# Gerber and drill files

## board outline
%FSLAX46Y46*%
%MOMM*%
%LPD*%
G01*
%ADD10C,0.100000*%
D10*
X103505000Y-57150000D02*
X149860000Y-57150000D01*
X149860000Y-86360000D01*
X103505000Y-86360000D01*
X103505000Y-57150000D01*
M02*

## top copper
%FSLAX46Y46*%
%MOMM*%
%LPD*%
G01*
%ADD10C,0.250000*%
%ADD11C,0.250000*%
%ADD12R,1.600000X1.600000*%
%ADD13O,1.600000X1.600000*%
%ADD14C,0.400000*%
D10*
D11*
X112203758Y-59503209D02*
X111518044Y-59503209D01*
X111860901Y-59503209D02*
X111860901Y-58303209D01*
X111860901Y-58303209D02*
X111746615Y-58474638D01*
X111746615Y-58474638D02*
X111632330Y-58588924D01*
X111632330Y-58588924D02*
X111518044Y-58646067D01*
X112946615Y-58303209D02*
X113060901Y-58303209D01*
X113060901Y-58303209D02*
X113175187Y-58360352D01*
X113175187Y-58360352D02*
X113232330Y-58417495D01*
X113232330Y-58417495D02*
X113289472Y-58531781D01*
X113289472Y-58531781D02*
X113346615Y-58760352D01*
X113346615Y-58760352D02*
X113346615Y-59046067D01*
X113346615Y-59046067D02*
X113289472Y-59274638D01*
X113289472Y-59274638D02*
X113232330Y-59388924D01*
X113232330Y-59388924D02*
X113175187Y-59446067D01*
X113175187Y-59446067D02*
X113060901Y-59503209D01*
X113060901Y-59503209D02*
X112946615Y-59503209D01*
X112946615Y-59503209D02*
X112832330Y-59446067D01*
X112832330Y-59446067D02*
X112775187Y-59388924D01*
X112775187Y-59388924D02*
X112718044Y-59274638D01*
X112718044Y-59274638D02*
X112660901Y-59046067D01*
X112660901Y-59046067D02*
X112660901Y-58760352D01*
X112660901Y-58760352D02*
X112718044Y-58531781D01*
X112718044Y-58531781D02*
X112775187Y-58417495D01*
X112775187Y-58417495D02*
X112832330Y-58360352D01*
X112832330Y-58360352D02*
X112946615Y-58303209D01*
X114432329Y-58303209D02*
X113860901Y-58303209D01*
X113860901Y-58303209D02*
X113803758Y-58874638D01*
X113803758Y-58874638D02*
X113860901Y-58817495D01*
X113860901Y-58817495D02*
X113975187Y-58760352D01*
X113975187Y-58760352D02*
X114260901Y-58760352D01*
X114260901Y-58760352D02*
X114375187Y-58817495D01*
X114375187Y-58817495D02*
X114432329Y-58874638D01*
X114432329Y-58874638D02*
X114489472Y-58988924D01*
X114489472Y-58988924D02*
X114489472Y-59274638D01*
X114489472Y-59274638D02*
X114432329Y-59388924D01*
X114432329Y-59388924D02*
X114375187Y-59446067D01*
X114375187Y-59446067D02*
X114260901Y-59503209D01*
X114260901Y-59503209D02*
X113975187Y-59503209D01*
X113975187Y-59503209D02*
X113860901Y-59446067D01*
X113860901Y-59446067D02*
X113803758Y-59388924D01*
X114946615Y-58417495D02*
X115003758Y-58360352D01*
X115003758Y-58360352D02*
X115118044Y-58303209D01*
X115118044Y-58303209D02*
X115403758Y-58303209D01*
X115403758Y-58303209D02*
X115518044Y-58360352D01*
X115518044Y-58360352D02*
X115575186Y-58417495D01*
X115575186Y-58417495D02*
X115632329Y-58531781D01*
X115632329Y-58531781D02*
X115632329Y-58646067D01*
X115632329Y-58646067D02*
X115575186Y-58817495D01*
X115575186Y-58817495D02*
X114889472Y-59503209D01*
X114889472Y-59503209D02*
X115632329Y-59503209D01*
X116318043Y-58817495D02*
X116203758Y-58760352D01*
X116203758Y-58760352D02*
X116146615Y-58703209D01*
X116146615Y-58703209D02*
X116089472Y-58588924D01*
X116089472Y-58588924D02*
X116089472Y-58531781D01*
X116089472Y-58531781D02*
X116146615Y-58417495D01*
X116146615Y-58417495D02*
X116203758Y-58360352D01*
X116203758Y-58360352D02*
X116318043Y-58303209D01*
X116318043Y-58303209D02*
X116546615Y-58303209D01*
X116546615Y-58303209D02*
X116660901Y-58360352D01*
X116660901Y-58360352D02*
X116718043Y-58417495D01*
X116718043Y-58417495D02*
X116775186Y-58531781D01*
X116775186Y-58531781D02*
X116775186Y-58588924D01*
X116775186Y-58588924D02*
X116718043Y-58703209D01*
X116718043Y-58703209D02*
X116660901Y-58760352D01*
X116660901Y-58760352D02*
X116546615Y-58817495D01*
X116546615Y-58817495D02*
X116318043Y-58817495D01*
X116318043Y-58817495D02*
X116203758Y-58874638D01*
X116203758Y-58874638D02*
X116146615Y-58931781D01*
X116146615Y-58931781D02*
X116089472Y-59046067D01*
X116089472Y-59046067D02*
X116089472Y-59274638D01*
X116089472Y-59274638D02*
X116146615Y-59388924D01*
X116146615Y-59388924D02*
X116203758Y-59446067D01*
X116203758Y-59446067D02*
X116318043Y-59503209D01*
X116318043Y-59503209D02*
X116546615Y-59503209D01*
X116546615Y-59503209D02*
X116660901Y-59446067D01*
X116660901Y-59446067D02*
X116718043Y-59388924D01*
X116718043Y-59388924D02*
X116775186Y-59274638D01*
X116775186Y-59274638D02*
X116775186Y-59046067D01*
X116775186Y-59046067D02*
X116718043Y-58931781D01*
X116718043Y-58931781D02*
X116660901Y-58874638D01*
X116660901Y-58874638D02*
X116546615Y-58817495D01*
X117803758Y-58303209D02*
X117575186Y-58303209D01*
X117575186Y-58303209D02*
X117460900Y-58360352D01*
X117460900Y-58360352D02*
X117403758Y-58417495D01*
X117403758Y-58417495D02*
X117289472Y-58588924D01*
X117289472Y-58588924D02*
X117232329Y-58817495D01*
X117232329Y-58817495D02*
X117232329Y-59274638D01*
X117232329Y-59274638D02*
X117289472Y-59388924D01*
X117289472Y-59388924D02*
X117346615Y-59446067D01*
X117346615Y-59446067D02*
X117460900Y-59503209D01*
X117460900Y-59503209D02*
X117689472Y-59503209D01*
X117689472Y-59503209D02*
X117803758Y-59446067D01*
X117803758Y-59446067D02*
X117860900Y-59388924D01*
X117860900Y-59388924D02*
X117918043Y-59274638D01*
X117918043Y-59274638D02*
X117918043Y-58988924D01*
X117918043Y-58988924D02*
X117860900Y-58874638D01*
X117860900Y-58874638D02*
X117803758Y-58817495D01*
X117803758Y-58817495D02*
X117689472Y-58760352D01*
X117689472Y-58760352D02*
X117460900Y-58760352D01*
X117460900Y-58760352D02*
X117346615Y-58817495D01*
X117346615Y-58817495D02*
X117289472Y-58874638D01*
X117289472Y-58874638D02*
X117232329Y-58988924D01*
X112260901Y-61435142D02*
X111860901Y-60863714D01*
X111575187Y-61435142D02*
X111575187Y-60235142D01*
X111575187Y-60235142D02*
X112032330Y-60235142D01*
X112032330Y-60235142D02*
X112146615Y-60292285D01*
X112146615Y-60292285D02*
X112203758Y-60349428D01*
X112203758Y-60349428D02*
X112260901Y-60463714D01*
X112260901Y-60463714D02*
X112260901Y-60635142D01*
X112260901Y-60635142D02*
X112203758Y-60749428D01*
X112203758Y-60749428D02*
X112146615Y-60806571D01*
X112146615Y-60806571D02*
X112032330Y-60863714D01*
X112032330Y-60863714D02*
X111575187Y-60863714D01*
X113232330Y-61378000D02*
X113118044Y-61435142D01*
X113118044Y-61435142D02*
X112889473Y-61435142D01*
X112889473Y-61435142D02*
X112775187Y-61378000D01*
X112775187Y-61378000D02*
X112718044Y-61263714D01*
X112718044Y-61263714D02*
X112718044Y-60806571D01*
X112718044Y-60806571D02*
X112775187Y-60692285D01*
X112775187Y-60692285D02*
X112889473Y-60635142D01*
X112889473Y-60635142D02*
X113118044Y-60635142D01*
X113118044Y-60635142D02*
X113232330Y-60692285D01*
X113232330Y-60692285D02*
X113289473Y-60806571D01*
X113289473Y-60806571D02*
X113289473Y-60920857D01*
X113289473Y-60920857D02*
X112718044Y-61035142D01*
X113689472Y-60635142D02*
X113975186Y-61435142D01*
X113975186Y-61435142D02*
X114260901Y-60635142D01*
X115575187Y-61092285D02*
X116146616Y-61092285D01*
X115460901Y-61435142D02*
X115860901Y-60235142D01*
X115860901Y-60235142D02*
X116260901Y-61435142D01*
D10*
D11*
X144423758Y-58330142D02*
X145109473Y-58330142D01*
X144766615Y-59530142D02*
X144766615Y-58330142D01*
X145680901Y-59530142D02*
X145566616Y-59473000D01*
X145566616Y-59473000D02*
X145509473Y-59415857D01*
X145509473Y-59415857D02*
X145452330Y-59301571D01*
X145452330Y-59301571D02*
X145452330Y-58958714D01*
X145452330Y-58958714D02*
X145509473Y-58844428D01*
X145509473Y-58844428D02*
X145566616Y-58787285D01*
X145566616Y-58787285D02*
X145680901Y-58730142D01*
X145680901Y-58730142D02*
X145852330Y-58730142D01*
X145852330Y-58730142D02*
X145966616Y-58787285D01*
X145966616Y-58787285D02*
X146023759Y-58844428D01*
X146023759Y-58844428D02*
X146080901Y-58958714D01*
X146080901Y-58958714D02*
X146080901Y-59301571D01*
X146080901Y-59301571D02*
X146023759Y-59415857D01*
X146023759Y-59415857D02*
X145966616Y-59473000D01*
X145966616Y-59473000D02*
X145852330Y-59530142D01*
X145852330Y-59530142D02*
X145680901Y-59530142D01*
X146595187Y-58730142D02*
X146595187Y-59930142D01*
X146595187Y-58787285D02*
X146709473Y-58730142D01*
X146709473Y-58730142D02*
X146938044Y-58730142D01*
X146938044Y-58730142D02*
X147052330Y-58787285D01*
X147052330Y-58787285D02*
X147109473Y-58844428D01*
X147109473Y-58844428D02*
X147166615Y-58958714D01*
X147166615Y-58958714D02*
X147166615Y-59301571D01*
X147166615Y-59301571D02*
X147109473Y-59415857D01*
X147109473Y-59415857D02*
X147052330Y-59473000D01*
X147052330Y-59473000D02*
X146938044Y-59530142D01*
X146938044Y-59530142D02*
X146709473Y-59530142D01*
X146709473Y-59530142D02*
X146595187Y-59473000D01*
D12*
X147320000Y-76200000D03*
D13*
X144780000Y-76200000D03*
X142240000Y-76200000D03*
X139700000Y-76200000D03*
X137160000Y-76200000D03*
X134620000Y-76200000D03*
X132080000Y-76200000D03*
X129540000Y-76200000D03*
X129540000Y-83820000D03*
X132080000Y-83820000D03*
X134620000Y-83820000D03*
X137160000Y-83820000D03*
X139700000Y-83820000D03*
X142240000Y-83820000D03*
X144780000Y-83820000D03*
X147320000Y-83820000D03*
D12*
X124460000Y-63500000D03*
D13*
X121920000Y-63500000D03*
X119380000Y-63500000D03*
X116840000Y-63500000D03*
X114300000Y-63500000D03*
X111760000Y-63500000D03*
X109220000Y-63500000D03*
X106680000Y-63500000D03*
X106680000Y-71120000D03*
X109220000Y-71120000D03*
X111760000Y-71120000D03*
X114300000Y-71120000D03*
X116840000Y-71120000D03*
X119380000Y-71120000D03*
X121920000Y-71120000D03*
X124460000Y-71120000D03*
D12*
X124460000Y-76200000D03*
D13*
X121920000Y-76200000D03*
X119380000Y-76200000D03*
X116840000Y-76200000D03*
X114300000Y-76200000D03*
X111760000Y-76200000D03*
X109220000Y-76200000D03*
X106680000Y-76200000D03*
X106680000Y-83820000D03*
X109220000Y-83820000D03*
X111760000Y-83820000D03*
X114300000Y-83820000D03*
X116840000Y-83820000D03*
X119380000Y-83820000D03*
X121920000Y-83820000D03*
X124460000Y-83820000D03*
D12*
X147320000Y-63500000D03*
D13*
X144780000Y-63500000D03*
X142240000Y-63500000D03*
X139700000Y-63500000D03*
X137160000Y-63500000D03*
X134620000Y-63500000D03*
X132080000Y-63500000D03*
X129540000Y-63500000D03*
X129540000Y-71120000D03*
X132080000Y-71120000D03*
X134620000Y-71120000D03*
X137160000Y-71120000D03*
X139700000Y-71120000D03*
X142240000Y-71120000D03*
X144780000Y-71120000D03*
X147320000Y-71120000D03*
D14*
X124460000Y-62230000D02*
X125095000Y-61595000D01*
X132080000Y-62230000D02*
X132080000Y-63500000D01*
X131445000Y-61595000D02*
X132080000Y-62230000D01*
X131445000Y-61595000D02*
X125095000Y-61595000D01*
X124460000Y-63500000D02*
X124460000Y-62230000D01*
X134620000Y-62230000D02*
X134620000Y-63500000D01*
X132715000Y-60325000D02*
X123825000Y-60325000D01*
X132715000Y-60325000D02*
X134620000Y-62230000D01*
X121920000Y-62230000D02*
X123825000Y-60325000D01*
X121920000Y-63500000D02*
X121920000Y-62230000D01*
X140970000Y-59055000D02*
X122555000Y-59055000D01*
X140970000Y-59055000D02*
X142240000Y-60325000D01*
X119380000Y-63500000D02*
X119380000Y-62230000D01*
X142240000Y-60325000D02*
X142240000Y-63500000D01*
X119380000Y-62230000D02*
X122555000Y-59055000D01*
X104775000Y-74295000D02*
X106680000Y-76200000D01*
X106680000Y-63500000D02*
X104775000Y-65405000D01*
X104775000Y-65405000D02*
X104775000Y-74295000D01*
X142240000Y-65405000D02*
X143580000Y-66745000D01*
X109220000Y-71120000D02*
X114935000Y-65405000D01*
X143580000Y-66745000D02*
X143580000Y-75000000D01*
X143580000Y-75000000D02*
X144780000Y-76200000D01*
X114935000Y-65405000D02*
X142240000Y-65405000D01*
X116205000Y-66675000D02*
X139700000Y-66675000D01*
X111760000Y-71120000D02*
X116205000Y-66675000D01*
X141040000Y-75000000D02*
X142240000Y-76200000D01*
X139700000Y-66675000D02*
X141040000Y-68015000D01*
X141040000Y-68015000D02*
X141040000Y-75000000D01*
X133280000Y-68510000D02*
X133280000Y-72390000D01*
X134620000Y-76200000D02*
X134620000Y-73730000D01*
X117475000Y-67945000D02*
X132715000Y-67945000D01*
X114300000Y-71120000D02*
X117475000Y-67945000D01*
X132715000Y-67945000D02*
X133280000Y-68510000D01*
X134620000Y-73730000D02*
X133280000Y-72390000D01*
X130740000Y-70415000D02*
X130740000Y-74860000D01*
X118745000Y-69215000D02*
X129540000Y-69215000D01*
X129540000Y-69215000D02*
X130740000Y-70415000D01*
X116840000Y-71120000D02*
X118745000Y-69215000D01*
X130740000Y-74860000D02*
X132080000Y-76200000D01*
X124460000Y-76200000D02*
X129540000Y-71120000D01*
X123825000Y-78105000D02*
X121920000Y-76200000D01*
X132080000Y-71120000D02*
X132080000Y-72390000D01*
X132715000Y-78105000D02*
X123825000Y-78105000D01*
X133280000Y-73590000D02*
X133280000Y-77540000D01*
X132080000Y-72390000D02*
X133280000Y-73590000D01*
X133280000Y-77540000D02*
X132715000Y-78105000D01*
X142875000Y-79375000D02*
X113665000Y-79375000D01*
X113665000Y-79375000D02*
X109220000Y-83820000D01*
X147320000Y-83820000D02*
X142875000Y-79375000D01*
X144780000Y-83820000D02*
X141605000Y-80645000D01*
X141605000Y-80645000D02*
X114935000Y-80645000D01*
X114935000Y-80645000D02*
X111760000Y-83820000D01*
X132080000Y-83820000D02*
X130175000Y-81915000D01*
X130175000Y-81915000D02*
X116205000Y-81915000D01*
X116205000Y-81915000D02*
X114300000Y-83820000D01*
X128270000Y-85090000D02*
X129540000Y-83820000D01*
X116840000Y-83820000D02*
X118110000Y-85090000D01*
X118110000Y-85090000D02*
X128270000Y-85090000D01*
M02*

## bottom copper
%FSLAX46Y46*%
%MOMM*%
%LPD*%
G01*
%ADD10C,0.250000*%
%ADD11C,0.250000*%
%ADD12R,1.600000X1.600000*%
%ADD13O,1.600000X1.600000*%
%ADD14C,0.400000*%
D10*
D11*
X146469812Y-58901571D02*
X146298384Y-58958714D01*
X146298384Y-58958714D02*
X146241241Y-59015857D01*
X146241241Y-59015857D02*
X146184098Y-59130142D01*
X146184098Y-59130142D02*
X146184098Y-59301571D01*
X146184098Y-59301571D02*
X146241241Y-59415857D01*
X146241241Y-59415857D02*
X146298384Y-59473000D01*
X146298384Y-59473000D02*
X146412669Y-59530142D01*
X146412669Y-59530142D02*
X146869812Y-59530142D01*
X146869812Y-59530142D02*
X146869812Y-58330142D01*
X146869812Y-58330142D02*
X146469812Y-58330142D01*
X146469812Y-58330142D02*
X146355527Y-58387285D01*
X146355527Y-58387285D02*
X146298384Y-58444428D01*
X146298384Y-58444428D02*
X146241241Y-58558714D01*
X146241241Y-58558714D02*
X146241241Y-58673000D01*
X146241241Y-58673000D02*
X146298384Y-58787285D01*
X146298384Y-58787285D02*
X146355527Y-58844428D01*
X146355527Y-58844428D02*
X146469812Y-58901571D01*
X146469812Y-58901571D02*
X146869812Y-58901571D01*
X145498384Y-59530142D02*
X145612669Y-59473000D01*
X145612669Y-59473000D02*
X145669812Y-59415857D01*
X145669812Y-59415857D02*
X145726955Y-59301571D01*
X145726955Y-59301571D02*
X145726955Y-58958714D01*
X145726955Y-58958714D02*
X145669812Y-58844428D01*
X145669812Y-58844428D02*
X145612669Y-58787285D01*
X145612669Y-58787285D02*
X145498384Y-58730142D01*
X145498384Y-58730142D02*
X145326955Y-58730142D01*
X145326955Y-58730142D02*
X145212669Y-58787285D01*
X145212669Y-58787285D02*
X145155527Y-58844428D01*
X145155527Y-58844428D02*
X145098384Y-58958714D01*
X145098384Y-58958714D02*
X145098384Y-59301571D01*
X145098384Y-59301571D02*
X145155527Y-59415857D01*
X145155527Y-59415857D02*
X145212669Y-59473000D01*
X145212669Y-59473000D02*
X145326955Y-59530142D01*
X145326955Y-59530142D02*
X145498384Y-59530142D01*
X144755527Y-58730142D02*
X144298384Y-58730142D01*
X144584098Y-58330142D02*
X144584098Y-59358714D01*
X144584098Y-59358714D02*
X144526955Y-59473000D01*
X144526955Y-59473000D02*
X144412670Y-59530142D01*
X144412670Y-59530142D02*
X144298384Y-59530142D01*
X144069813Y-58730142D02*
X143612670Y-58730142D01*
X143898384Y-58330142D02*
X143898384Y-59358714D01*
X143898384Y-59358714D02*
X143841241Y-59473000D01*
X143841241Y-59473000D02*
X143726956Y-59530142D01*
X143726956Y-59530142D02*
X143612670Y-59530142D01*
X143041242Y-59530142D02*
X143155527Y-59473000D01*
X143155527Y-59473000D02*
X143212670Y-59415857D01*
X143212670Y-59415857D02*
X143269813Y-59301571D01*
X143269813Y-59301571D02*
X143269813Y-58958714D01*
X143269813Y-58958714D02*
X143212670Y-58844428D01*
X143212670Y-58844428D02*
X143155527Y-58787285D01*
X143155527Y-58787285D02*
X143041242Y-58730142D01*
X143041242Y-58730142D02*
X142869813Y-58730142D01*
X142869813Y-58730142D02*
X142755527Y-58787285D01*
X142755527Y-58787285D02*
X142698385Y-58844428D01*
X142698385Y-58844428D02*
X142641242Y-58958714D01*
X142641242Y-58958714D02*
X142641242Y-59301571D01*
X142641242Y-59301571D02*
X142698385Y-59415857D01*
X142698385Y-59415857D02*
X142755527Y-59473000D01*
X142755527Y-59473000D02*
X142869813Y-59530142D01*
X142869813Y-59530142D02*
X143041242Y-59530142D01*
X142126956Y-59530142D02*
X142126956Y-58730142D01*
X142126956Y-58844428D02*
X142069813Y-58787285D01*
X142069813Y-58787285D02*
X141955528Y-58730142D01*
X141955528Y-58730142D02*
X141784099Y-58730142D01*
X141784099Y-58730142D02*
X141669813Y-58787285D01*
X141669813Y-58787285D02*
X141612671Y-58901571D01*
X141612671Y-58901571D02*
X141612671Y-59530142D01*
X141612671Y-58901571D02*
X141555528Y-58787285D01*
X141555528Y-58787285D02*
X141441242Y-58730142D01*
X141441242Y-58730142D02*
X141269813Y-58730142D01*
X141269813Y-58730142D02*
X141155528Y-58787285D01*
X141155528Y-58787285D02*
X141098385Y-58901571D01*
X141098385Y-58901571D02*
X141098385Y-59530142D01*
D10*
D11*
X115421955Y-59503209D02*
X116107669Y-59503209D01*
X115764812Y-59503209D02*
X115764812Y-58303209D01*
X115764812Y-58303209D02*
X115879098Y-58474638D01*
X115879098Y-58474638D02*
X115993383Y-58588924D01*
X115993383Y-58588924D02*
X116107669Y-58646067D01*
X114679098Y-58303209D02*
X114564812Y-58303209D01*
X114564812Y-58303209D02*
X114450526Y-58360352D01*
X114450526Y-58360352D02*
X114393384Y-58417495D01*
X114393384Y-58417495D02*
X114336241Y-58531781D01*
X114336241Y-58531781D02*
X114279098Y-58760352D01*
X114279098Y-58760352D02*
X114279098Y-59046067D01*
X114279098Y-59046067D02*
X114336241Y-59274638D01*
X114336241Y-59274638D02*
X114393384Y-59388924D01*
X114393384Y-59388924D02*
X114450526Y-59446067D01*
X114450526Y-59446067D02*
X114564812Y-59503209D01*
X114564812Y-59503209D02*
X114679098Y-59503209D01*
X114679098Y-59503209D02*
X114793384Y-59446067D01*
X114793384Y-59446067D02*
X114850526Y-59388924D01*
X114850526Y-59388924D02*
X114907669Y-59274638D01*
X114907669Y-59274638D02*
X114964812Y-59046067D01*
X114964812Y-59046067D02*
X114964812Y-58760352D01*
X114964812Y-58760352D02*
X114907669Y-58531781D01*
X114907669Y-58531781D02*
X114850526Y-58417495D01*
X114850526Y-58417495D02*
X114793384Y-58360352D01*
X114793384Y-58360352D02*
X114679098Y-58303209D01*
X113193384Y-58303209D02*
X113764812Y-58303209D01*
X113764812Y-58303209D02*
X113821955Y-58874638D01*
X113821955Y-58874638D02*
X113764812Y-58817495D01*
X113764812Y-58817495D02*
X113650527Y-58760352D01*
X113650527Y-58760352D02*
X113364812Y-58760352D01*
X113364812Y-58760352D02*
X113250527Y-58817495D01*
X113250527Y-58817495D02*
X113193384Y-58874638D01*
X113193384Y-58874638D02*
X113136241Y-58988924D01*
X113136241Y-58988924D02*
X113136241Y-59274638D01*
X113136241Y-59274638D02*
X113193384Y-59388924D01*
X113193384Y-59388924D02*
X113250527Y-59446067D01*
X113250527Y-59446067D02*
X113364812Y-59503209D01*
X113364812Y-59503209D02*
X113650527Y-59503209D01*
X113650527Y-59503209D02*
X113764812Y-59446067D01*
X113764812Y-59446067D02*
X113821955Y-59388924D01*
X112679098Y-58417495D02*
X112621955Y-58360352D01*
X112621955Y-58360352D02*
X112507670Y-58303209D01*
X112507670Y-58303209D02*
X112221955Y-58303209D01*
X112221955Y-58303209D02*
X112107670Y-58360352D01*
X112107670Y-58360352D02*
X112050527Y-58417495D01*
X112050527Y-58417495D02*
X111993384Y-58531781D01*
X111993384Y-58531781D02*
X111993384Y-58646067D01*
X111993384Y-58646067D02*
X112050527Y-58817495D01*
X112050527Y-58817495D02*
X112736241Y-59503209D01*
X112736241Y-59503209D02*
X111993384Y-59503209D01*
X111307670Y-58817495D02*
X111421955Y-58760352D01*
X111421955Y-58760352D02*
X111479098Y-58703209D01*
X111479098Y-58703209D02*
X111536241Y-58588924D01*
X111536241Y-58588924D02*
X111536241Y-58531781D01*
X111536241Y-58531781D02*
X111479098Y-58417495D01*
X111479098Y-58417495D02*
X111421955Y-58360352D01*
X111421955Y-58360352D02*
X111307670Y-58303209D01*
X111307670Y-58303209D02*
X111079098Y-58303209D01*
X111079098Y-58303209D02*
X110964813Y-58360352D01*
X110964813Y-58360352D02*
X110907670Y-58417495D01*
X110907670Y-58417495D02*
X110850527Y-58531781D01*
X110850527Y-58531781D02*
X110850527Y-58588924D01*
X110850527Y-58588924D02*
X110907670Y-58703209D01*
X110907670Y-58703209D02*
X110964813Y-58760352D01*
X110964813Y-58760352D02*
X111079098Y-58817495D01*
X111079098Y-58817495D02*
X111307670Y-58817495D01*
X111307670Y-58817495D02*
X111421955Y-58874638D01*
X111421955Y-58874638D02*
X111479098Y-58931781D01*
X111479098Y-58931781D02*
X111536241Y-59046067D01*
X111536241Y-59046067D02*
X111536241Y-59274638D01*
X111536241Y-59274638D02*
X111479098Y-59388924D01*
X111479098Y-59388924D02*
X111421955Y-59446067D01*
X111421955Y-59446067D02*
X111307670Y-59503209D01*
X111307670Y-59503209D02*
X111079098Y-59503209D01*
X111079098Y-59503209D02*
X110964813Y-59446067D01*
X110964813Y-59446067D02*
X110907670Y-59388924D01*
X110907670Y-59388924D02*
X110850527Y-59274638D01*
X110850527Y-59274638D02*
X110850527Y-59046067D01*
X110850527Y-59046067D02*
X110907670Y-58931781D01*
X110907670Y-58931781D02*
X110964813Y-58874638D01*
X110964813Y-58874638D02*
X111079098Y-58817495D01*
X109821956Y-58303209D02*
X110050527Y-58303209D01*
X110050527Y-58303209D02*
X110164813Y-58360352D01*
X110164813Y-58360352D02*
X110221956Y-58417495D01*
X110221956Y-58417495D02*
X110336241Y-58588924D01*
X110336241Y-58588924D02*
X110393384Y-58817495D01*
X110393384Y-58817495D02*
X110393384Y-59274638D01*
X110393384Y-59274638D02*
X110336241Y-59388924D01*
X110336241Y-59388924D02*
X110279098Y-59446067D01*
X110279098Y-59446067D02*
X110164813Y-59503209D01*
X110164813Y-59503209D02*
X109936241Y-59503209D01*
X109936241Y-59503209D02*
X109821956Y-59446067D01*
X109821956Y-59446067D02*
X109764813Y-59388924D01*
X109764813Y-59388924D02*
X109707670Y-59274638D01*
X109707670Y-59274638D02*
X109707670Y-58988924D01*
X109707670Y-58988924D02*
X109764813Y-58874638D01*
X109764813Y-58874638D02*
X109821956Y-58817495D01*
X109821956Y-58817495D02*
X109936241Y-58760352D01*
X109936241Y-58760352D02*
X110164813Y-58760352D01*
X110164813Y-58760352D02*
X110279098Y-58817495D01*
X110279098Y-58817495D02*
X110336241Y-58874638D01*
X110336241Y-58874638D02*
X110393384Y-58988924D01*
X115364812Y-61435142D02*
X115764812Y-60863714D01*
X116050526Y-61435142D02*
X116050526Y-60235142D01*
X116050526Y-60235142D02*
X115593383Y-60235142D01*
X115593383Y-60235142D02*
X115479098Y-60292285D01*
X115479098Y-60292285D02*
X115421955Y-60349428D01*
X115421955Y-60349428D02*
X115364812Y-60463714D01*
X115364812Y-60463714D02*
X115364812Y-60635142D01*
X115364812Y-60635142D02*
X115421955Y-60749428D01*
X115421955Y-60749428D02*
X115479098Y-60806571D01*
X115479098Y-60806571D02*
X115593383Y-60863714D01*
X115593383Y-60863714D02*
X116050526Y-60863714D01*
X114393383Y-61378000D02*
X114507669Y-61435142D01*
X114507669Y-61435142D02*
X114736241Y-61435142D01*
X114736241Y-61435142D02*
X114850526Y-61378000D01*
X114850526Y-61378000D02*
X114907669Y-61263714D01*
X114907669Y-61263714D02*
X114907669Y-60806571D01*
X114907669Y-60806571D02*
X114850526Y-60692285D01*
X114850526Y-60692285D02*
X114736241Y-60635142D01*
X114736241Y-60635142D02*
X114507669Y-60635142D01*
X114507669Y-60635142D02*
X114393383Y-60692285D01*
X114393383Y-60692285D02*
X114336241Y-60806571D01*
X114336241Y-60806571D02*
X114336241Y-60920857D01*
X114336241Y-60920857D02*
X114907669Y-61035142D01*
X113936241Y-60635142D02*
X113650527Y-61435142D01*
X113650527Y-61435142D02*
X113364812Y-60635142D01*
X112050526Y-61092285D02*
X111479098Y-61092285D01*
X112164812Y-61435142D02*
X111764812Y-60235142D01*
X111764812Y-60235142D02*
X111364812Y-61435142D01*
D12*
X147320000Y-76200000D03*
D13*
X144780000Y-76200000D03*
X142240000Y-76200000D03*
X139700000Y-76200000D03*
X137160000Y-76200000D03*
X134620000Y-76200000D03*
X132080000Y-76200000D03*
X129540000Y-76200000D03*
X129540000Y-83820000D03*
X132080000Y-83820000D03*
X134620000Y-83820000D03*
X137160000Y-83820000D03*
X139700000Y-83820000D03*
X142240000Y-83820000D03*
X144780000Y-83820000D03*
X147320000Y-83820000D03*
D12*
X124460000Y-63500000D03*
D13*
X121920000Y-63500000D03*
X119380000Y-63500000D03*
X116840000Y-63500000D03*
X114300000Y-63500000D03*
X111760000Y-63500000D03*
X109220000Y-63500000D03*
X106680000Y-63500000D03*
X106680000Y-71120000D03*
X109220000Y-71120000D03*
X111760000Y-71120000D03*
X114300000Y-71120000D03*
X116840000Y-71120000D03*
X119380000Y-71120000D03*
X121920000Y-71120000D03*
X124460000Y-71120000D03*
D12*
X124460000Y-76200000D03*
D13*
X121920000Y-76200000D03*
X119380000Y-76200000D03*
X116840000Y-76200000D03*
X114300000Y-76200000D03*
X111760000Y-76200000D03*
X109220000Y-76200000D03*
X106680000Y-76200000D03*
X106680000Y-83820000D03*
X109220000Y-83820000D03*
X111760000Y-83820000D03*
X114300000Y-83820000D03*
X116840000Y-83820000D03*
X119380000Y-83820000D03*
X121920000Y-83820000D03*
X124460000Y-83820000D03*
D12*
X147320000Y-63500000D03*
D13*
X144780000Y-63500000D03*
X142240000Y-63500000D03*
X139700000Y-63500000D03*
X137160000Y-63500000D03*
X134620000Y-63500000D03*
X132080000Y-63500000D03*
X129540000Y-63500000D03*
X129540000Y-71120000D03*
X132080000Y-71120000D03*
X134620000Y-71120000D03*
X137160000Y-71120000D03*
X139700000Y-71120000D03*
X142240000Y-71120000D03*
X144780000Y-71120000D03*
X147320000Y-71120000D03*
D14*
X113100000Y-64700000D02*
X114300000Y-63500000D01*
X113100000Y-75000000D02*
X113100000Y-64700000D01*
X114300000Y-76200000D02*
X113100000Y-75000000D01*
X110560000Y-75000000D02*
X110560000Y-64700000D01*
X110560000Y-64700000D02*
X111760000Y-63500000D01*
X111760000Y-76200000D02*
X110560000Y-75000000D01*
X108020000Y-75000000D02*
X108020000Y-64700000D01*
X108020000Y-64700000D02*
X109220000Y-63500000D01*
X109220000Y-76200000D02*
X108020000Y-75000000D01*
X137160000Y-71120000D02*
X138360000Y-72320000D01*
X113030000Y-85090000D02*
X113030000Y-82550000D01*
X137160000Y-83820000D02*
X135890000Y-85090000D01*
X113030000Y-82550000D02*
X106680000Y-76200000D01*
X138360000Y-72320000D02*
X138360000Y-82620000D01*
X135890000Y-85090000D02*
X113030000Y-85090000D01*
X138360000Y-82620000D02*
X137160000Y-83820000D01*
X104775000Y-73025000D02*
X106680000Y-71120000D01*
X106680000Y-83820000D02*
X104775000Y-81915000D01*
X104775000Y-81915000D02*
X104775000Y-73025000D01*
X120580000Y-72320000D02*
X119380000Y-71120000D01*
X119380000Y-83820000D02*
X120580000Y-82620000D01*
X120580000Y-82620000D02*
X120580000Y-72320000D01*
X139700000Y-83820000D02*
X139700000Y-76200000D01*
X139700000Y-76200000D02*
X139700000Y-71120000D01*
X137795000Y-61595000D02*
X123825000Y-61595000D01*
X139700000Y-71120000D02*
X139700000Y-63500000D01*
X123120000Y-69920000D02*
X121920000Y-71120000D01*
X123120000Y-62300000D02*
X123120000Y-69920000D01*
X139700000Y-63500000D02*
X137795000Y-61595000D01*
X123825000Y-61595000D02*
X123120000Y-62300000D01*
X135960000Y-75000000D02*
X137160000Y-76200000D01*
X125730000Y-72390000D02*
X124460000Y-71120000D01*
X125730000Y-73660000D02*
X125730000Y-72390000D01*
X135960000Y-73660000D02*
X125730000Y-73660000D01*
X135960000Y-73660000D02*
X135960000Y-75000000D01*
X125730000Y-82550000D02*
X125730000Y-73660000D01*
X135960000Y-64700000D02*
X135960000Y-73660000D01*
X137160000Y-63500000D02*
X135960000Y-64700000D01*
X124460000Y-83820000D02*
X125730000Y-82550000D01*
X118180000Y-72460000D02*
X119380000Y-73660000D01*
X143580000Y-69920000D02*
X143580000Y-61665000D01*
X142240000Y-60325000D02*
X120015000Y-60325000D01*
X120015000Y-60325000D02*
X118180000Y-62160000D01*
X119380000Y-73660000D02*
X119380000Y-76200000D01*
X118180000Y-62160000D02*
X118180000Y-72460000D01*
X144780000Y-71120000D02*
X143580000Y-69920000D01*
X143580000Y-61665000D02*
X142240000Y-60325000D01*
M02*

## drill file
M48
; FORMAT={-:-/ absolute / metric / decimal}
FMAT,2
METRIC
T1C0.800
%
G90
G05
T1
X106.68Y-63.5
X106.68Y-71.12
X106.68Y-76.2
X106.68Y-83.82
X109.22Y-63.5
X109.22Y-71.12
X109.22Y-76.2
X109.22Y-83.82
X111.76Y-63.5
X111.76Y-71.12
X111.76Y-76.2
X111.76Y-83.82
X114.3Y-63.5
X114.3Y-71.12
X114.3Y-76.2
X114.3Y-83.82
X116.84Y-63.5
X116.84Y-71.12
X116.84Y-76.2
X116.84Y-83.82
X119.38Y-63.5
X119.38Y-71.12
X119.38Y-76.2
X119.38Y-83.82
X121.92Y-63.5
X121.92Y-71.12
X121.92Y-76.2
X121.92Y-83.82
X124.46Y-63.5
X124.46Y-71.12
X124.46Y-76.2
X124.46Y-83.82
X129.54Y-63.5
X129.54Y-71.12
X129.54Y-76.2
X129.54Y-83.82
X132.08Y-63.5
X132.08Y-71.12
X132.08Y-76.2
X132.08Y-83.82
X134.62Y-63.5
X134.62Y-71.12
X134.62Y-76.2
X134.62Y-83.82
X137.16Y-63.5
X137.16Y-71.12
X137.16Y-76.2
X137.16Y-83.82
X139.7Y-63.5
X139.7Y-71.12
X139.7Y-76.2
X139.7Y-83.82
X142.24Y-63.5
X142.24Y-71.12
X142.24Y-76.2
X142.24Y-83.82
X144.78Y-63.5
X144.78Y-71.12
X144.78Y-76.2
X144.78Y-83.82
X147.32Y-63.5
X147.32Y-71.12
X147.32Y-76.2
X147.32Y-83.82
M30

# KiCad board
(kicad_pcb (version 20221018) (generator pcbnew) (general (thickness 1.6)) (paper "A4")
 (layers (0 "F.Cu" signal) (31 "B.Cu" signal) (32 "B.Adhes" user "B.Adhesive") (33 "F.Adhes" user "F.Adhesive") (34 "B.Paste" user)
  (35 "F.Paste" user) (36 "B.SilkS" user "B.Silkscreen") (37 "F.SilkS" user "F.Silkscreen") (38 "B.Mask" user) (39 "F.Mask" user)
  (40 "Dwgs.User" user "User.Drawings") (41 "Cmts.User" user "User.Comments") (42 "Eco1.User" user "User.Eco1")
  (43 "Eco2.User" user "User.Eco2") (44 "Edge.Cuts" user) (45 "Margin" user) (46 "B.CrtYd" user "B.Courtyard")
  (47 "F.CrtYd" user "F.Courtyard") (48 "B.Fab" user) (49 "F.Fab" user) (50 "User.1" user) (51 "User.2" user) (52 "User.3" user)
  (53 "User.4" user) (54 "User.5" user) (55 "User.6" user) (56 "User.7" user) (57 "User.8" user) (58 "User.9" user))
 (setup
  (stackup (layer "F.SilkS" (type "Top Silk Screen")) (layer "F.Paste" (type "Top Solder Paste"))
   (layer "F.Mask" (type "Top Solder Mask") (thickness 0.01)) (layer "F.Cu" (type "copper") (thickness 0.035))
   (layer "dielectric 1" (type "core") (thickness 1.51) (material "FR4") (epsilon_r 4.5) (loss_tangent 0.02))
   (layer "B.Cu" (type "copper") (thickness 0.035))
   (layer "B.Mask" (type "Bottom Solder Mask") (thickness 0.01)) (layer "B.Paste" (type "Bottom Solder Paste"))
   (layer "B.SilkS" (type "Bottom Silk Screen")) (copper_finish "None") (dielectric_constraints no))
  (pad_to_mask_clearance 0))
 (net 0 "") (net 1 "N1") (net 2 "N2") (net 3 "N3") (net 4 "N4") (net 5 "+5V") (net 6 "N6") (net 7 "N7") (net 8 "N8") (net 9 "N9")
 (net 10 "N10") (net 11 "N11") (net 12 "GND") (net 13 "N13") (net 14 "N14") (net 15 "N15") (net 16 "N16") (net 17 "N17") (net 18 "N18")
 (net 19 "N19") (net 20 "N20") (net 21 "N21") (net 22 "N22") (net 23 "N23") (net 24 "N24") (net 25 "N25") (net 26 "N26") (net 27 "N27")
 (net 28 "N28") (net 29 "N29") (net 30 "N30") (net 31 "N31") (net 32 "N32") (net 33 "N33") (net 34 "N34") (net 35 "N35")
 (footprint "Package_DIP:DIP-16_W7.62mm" (layer "F.Cu") (at 147.32 76.2 -90)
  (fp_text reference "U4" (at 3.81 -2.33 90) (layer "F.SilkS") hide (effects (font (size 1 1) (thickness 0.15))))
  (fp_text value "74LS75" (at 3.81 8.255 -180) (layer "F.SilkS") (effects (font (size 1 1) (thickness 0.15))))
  (pad "1" thru_hole rect (at 0 0 270) (size 1.6 1.6) (drill 0.8) (layers "*.Cu" "*.Mask") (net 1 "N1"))
  (pad "2" thru_hole oval (at 0 2.54 270) (size 1.6 1.6) (drill 0.8) (layers "*.Cu" "*.Mask") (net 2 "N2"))
  (pad "3" thru_hole oval (at 0 5.08 270) (size 1.6 1.6) (drill 0.8) (layers "*.Cu" "*.Mask") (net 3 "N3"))
  (pad "4" thru_hole oval (at 0 7.62 270) (size 1.6 1.6) (drill 0.8) (layers "*.Cu" "*.Mask") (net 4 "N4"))
  (pad "5" thru_hole oval (at 0 10.16 270) (size 1.6 1.6) (drill 0.8) (layers "*.Cu" "*.Mask") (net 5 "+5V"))
  (pad "6" thru_hole oval (at 0 12.7 270) (size 1.6 1.6) (drill 0.8) (layers "*.Cu" "*.Mask") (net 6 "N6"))
  (pad "7" thru_hole oval (at 0 15.24 270) (size 1.6 1.6) (drill 0.8) (layers "*.Cu" "*.Mask") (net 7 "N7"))
  (pad "8" thru_hole oval (at 0 17.78 270) (size 1.6 1.6) (drill 0.8) (layers "*.Cu" "*.Mask") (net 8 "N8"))
  (pad "9" thru_hole oval (at 7.62 17.78 270) (size 1.6 1.6) (drill 0.8) (layers "*.Cu" "*.Mask") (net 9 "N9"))
  (pad "10" thru_hole oval (at 7.62 15.24 270) (size 1.6 1.6) (drill 0.8) (layers "*.Cu" "*.Mask") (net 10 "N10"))
  (pad "11" thru_hole oval (at 7.62 12.7 270) (size 1.6 1.6) (drill 0.8) (layers "*.Cu" "*.Mask") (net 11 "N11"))
  (pad "12" thru_hole oval (at 7.62 10.16 270) (size 1.6 1.6) (drill 0.8) (layers "*.Cu" "*.Mask") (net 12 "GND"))
  (pad "13" thru_hole oval (at 7.62 7.62 270) (size 1.6 1.6) (drill 0.8) (layers "*.Cu" "*.Mask") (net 4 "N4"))
  (pad "14" thru_hole oval (at 7.62 5.08 270) (size 1.6 1.6) (drill 0.8) (layers "*.Cu" "*.Mask") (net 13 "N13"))
  (pad "15" thru_hole oval (at 7.62 2.54 270) (size 1.6 1.6) (drill 0.8) (layers "*.Cu" "*.Mask") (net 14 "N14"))
  (pad "16" thru_hole oval (at 7.62 0 270) (size 1.6 1.6) (drill 0.8) (layers "*.Cu" "*.Mask") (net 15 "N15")))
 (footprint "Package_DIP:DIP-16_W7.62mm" (layer "F.Cu") (at 124.46 63.5 -90)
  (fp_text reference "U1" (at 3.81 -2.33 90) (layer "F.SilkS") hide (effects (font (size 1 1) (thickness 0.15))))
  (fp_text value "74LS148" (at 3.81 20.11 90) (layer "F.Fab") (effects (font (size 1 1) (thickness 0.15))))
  (pad "1" thru_hole rect (at 0 0 270) (size 1.6 1.6) (drill 0.8) (layers "*.Cu" "*.Mask") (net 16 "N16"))
  (pad "2" thru_hole oval (at 0 2.54 270) (size 1.6 1.6) (drill 0.8) (layers "*.Cu" "*.Mask") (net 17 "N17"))
  (pad "3" thru_hole oval (at 0 5.08 270) (size 1.6 1.6) (drill 0.8) (layers "*.Cu" "*.Mask") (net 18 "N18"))
  (pad "4" thru_hole oval (at 0 7.62 270) (size 1.6 1.6) (drill 0.8) (layers "*.Cu" "*.Mask") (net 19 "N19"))
  (pad "5" thru_hole oval (at 0 10.16 270) (size 1.6 1.6) (drill 0.8) (layers "*.Cu" "*.Mask") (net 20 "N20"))
  (pad "6" thru_hole oval (at 0 12.7 270) (size 1.6 1.6) (drill 0.8) (layers "*.Cu" "*.Mask") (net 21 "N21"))
  (pad "7" thru_hole oval (at 0 15.24 270) (size 1.6 1.6) (drill 0.8) (layers "*.Cu" "*.Mask") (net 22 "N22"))
  (pad "8" thru_hole oval (at 0 17.78 270) (size 1.6 1.6) (drill 0.8) (layers "*.Cu" "*.Mask") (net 12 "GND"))
  (pad "9" thru_hole oval (at 7.62 17.78 270) (size 1.6 1.6) (drill 0.8) (layers "*.Cu" "*.Mask") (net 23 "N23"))
  (pad "10" thru_hole oval (at 7.62 15.24 270) (size 1.6 1.6) (drill 0.8) (layers "*.Cu" "*.Mask") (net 2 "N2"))
  (pad "11" thru_hole oval (at 7.62 12.7 270) (size 1.6 1.6) (drill 0.8) (layers "*.Cu" "*.Mask") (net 3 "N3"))
  (pad "12" thru_hole oval (at 7.62 10.16 270) (size 1.6 1.6) (drill 0.8) (layers "*.Cu" "*.Mask") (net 6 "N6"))
  (pad "13" thru_hole oval (at 7.62 7.62 270) (size 1.6 1.6) (drill 0.8) (layers "*.Cu" "*.Mask") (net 7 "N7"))
  (pad "14" thru_hole oval (at 7.62 5.08 270) (size 1.6 1.6) (drill 0.8) (layers "*.Cu" "*.Mask") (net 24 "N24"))
  (pad "15" thru_hole oval (at 7.62 2.54 270) (size 1.6 1.6) (drill 0.8) (layers "*.Cu" "*.Mask") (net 4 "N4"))
  (pad "16" thru_hole oval (at 7.62 0 270) (size 1.6 1.6) (drill 0.8) (layers "*.Cu" "*.Mask") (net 5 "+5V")))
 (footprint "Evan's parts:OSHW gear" (layer "F.Cu") (at 108.585 80.01)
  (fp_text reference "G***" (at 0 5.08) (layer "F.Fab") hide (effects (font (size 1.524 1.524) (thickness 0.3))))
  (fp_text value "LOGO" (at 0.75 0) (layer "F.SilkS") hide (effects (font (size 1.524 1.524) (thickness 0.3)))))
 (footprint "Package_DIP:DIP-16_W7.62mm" (layer "F.Cu") (at 124.46 76.2 -90)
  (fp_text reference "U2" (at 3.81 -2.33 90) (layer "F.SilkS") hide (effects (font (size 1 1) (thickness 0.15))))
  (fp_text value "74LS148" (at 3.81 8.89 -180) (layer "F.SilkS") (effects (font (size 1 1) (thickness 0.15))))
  (pad "1" thru_hole rect (at 0 0 270) (size 1.6 1.6) (drill 0.8) (layers "*.Cu" "*.Mask") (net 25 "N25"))
  (pad "2" thru_hole oval (at 0 2.54 270) (size 1.6 1.6) (drill 0.8) (layers "*.Cu" "*.Mask") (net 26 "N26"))
  (pad "3" thru_hole oval (at 0 5.08 270) (size 1.6 1.6) (drill 0.8) (layers "*.Cu" "*.Mask") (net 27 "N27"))
  (pad "4" thru_hole oval (at 0 7.62 270) (size 1.6 1.6) (drill 0.8) (layers "*.Cu" "*.Mask") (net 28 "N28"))
  (pad "5" thru_hole oval (at 0 10.16 270) (size 1.6 1.6) (drill 0.8) (layers "*.Cu" "*.Mask") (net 20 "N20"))
  (pad "6" thru_hole oval (at 0 12.7 270) (size 1.6 1.6) (drill 0.8) (layers "*.Cu" "*.Mask") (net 21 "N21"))
  (pad "7" thru_hole oval (at 0 15.24 270) (size 1.6 1.6) (drill 0.8) (layers "*.Cu" "*.Mask") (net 22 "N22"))
  (pad "8" thru_hole oval (at 0 17.78 270) (size 1.6 1.6) (drill 0.8) (layers "*.Cu" "*.Mask") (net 12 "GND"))
  (pad "9" thru_hole oval (at 7.62 17.78 270) (size 1.6 1.6) (drill 0.8) (layers "*.Cu" "*.Mask") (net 23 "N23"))
  (pad "10" thru_hole oval (at 7.62 15.24 270) (size 1.6 1.6) (drill 0.8) (layers "*.Cu" "*.Mask") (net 15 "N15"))
  (pad "11" thru_hole oval (at 7.62 12.7 270) (size 1.6 1.6) (drill 0.8) (layers "*.Cu" "*.Mask") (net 14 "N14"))
  (pad "12" thru_hole oval (at 7.62 10.16 270) (size 1.6 1.6) (drill 0.8) (layers "*.Cu" "*.Mask") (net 10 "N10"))
  (pad "13" thru_hole oval (at 7.62 7.62 270) (size 1.6 1.6) (drill 0.8) (layers "*.Cu" "*.Mask") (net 9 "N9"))
  (pad "14" thru_hole oval (at 7.62 5.08 270) (size 1.6 1.6) (drill 0.8) (layers "*.Cu" "*.Mask") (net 24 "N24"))
  (pad "15" thru_hole oval (at 7.62 2.54 270) (size 1.6 1.6) (drill 0.8) (layers "*.Cu" "*.Mask") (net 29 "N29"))
  (pad "16" thru_hole oval (at 7.62 0 270) (size 1.6 1.6) (drill 0.8) (layers "*.Cu" "*.Mask") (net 5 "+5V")))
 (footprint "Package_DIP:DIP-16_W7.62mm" (layer "F.Cu") (at 147.32 63.5 -90)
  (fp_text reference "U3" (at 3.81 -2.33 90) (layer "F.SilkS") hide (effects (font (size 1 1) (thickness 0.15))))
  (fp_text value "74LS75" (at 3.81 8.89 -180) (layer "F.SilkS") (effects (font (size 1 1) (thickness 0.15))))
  (pad "1" thru_hole rect (at 0 0 270) (size 1.6 1.6) (drill 0.8) (layers "*.Cu" "*.Mask") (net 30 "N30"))
  (pad "2" thru_hole oval (at 0 2.54 270) (size 1.6 1.6) (drill 0.8) (layers "*.Cu" "*.Mask") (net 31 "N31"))
  (pad "3" thru_hole oval (at 0 5.08 270) (size 1.6 1.6) (drill 0.8) (layers "*.Cu" "*.Mask") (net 18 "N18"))
  (pad "4" thru_hole oval (at 0 7.62 270) (size 1.6 1.6) (drill 0.8) (layers "*.Cu" "*.Mask") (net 4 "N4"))
  (pad "5" thru_hole oval (at 0 10.16 270) (size 1.6 1.6) (drill 0.8) (layers "*.Cu" "*.Mask") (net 5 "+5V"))
  (pad "6" thru_hole oval (at 0 12.7 270) (size 1.6 1.6) (drill 0.8) (layers "*.Cu" "*.Mask") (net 17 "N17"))
  (pad "7" thru_hole oval (at 0 15.24 270) (size 1.6 1.6) (drill 0.8) (layers "*.Cu" "*.Mask") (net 16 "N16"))
  (pad "8" thru_hole oval (at 0 17.78 270) (size 1.6 1.6) (drill 0.8) (layers "*.Cu" "*.Mask") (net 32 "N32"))
  (pad "9" thru_hole oval (at 7.62 17.78 270) (size 1.6 1.6) (drill 0.8) (layers "*.Cu" "*.Mask") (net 25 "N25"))
  (pad "10" thru_hole oval (at 7.62 15.24 270) (size 1.6 1.6) (drill 0.8) (layers "*.Cu" "*.Mask") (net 26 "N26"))
  (pad "11" thru_hole oval (at 7.62 12.7 270) (size 1.6 1.6) (drill 0.8) (layers "*.Cu" "*.Mask") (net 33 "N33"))
  (pad "12" thru_hole oval (at 7.62 10.16 270) (size 1.6 1.6) (drill 0.8) (layers "*.Cu" "*.Mask") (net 12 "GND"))
  (pad "13" thru_hole oval (at 7.62 7.62 270) (size 1.6 1.6) (drill 0.8) (layers "*.Cu" "*.Mask") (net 4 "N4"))
  (pad "14" thru_hole oval (at 7.62 5.08 270) (size 1.6 1.6) (drill 0.8) (layers "*.Cu" "*.Mask") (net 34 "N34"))
  (pad "15" thru_hole oval (at 7.62 2.54 270) (size 1.6 1.6) (drill 0.8) (layers "*.Cu" "*.Mask") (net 27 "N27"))
  (pad "16" thru_hole oval (at 7.62 0 270) (size 1.6 1.6) (drill 0.8) (layers "*.Cu" "*.Mask") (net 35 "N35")))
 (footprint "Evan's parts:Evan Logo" (layer "B.Cu") (at 144.145 67.31 180)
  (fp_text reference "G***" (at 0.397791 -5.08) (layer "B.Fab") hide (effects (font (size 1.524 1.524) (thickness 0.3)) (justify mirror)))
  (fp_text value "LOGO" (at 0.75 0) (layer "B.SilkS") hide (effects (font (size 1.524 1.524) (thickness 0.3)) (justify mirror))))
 (gr_rect (start 103.505 57.15) (end 149.86 86.36) (stroke (width 0.1) (type default)) (fill none) (layer "Edge.Cuts"))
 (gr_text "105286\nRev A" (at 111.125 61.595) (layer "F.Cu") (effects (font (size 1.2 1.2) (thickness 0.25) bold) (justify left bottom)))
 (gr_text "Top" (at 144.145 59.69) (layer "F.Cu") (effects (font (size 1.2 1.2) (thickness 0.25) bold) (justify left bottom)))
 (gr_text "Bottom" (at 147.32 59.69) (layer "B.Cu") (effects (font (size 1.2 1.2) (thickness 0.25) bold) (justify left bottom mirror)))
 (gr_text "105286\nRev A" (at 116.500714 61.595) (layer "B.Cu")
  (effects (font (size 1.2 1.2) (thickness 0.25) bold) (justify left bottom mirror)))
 (segment (start 124.46 62.23) (end 125.095 61.595) (width 0.4) (layer "F.Cu") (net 16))
 (segment (start 132.08 62.23) (end 132.08 63.5) (width 0.4) (layer "F.Cu") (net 16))
 (segment (start 131.445 61.595) (end 132.08 62.23) (width 0.4) (layer "F.Cu") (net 16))
 (segment (start 131.445 61.595) (end 125.095 61.595) (width 0.4) (layer "F.Cu") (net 16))
 (segment (start 124.46 63.5) (end 124.46 62.23) (width 0.4) (layer "F.Cu") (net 16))
 (segment (start 134.62 62.23) (end 134.62 63.5) (width 0.4) (layer "F.Cu") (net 17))
 (segment (start 132.715 60.325) (end 123.825 60.325) (width 0.4) (layer "F.Cu") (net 17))
 (segment (start 132.715 60.325) (end 134.62 62.23) (width 0.4) (layer "F.Cu") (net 17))
 (segment (start 121.92 62.23) (end 123.825 60.325) (width 0.4) (layer "F.Cu") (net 17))
 (segment (start 121.92 63.5) (end 121.92 62.23) (width 0.4) (layer "F.Cu") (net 17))
 (segment (start 140.97 59.055) (end 122.555 59.055) (width 0.4) (layer "F.Cu") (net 18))
 (segment (start 140.97 59.055) (end 142.24 60.325) (width 0.4) (layer "F.Cu") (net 18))
 (segment (start 119.38 63.5) (end 119.38 62.23) (width 0.4) (layer "F.Cu") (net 18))
 (segment (start 142.24 60.325) (end 142.24 63.5) (width 0.4) (layer "F.Cu") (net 18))
 (segment (start 119.38 62.23) (end 122.555 59.055) (width 0.4) (layer "F.Cu") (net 18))
 (segment (start 113.1 64.7) (end 114.3 63.5) (width 0.4) (layer "B.Cu") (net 20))
 (segment (start 113.1 75) (end 113.1 64.7) (width 0.4) (layer "B.Cu") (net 20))
 (segment (start 114.3 76.2) (end 113.1 75) (width 0.4) (layer "B.Cu") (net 20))
 (segment (start 110.56 75) (end 110.56 64.7) (width 0.4) (layer "B.Cu") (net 21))
 (segment (start 110.56 64.7) (end 111.76 63.5) (width 0.4) (layer "B.Cu") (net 21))
 (segment (start 111.76 76.2) (end 110.56 75) (width 0.4) (layer "B.Cu") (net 21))
 (segment (start 108.02 75) (end 108.02 64.7) (width 0.4) (layer "B.Cu") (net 22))
 (segment (start 108.02 64.7) (end 109.22 63.5) (width 0.4) (layer "B.Cu") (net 22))
 (segment (start 109.22 76.2) (end 108.02 75) (width 0.4) (layer "B.Cu") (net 22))
 (segment (start 104.775 74.295) (end 106.68 76.2) (width 0.4) (layer "F.Cu") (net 12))
 (segment (start 106.68 63.5) (end 104.775 65.405) (width 0.4) (layer "F.Cu") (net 12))
 (segment (start 104.775 65.405) (end 104.775 74.295) (width 0.4) (layer "F.Cu") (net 12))
 (segment (start 137.16 71.12) (end 138.36 72.32) (width 0.4) (layer "B.Cu") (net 12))
 (segment (start 113.03 85.09) (end 113.03 82.55) (width 0.4) (layer "B.Cu") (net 12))
 (segment (start 137.16 83.82) (end 135.89 85.09) (width 0.4) (layer "B.Cu") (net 12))
 (segment (start 113.03 82.55) (end 106.68 76.2) (width 0.4) (layer "B.Cu") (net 12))
 (segment (start 138.36 72.32) (end 138.36 82.62) (width 0.4) (layer "B.Cu") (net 12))
 (segment (start 135.89 85.09) (end 113.03 85.09) (width 0.4) (layer "B.Cu") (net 12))
 (segment (start 138.36 82.62) (end 137.16 83.82) (width 0.4) (layer "B.Cu") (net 12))
 (segment (start 104.775 73.025) (end 106.68 71.12) (width 0.4) (layer "B.Cu") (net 23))
 (segment (start 106.68 83.82) (end 104.775 81.915) (width 0.4) (layer "B.Cu") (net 23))
 (segment (start 104.775 81.915) (end 104.775 73.025) (width 0.4) (layer "B.Cu") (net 23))
 (segment (start 142.24 65.405) (end 143.58 66.745) (width 0.4) (layer "F.Cu") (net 2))
 (segment (start 109.22 71.12) (end 114.935 65.405) (width 0.4) (layer "F.Cu") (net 2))
 (segment (start 143.58 66.745) (end 143.58 75) (width 0.4) (layer "F.Cu") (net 2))
 (segment (start 143.58 75) (end 144.78 76.2) (width 0.4) (layer "F.Cu") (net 2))
 (segment (start 114.935 65.405) (end 142.24 65.405) (width 0.4) (layer "F.Cu") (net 2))
 (segment (start 116.205 66.675) (end 139.7 66.675) (width 0.4) (layer "F.Cu") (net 3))
 (segment (start 111.76 71.12) (end 116.205 66.675) (width 0.4) (layer "F.Cu") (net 3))
 (segment (start 141.04 75) (end 142.24 76.2) (width 0.4) (layer "F.Cu") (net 3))
 (segment (start 139.7 66.675) (end 141.04 68.015) (width 0.4) (layer "F.Cu") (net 3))
 (segment (start 141.04 68.015) (end 141.04 75) (width 0.4) (layer "F.Cu") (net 3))
 (segment (start 133.28 68.51) (end 133.28 72.39) (width 0.4) (layer "F.Cu") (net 6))
 (segment (start 134.62 76.2) (end 134.62 73.73) (width 0.4) (layer "F.Cu") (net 6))
 (segment (start 117.475 67.945) (end 132.715 67.945) (width 0.4) (layer "F.Cu") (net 6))
 (segment (start 114.3 71.12) (end 117.475 67.945) (width 0.4) (layer "F.Cu") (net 6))
 (segment (start 132.715 67.945) (end 133.28 68.51) (width 0.4) (layer "F.Cu") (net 6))
 (segment (start 134.62 73.73) (end 133.28 72.39) (width 0.4) (layer "F.Cu") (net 6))
 (segment (start 130.74 70.415) (end 130.74 74.86) (width 0.4) (layer "F.Cu") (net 7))
 (segment (start 118.745 69.215) (end 129.54 69.215) (width 0.4) (layer "F.Cu") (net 7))
 (segment (start 129.54 69.215) (end 130.74 70.415) (width 0.4) (layer "F.Cu") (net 7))
 (segment (start 116.84 71.12) (end 118.745 69.215) (width 0.4) (layer "F.Cu") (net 7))
 (segment (start 130.74 74.86) (end 132.08 76.2) (width 0.4) (layer "F.Cu") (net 7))
 (segment (start 120.58 72.32) (end 119.38 71.12) (width 0.4) (layer "B.Cu") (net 24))
 (segment (start 119.38 83.82) (end 120.58 82.62) (width 0.4) (layer "B.Cu") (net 24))
 (segment (start 120.58 82.62) (end 120.58 72.32) (width 0.4) (layer "B.Cu") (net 24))
 (segment (start 139.7 83.82) (end 139.7 76.2) (width 0.4) (layer "B.Cu") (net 4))
 (segment (start 139.7 76.2) (end 139.7 71.12) (width 0.4) (layer "B.Cu") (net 4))
 (segment (start 137.795 61.595) (end 123.825 61.595) (width 0.4) (layer "B.Cu") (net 4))
 (segment (start 139.7 71.12) (end 139.7 63.5) (width 0.4) (layer "B.Cu") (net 4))
 (segment (start 123.12 69.92) (end 121.92 71.12) (width 0.4) (layer "B.Cu") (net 4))
 (segment (start 123.12 62.3) (end 123.12 69.92) (width 0.4) (layer "B.Cu") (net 4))
 (segment (start 139.7 63.5) (end 137.795 61.595) (width 0.4) (layer "B.Cu") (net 4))
 (segment (start 123.825 61.595) (end 123.12 62.3) (width 0.4) (layer "B.Cu") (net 4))
 (segment (start 135.96 75) (end 137.16 76.2) (width 0.4) (layer "B.Cu") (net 5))
 (segment (start 125.73 72.39) (end 124.46 71.12) (width 0.4) (layer "B.Cu") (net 5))
 (segment (start 125.73 73.66) (end 125.73 72.39) (width 0.4) (layer "B.Cu") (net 5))
 (segment (start 135.96 73.66) (end 125.73 73.66) (width 0.4) (layer "B.Cu") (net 5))
 (segment (start 135.96 73.66) (end 135.96 75) (width 0.4) (layer "B.Cu") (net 5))
 (segment (start 125.73 82.55) (end 125.73 73.66) (width 0.4) (layer "B.Cu") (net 5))
 (segment (start 135.96 64.7) (end 135.96 73.66) (width 0.4) (layer "B.Cu") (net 5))
 (segment (start 137.16 63.5) (end 135.96 64.7) (width 0.4) (layer "B.Cu") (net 5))
 (segment (start 124.46 83.82) (end 125.73 82.55) (width 0.4) (layer "B.Cu") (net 5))
 (segment (start 124.46 76.2) (end 129.54 71.12) (width 0.4) (layer "F.Cu") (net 25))
 (segment (start 123.825 78.105) (end 121.92 76.2) (width 0.4) (layer "F.Cu") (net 26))
 (segment (start 132.08 71.12) (end 132.08 72.39) (width 0.4) (layer "F.Cu") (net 26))
 (segment (start 132.715 78.105) (end 123.825 78.105) (width 0.4) (layer "F.Cu") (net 26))
 (segment (start 133.28 73.59) (end 133.28 77.54) (width 0.4) (layer "F.Cu") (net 26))
 (segment (start 132.08 72.39) (end 133.28 73.59) (width 0.4) (layer "F.Cu") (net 26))
 (segment (start 133.28 77.54) (end 132.715 78.105) (width 0.4) (layer "F.Cu") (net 26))
 (segment (start 118.18 72.46) (end 119.38 73.66) (width 0.4) (layer "B.Cu") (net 27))
 (segment (start 143.58 69.92) (end 143.58 61.665) (width 0.4) (layer "B.Cu") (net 27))
 (segment (start 142.24 60.325) (end 120.015 60.325) (width 0.4) (layer "B.Cu") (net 27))
 (segment (start 120.015 60.325) (end 118.18 62.16) (width 0.4) (layer "B.Cu") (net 27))
 (segment (start 119.38 73.66) (end 119.38 76.2) (width 0.4) (layer "B.Cu") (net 27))
 (segment (start 118.18 62.16) (end 118.18 72.46) (width 0.4) (layer "B.Cu") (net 27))
 (segment (start 144.78 71.12) (end 143.58 69.92) (width 0.4) (layer "B.Cu") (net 27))
 (segment (start 143.58 61.665) (end 142.24 60.325) (width 0.4) (layer "B.Cu") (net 27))
 (segment (start 142.875 79.375) (end 113.665 79.375) (width 0.4) (layer "F.Cu") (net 15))
 (segment (start 113.665 79.375) (end 109.22 83.82) (width 0.4) (layer "F.Cu") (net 15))
 (segment (start 147.32 83.82) (end 142.875 79.375) (width 0.4) (layer "F.Cu") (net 15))
 (segment (start 144.78 83.82) (end 141.605 80.645) (width 0.4) (layer "F.Cu") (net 14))
 (segment (start 141.605 80.645) (end 114.935 80.645) (width 0.4) (layer "F.Cu") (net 14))
 (segment (start 114.935 80.645) (end 111.76 83.82) (width 0.4) (layer "F.Cu") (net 14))
 (segment (start 132.08 83.82) (end 130.175 81.915) (width 0.4) (layer "F.Cu") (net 10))
 (segment (start 130.175 81.915) (end 116.205 81.915) (width 0.4) (layer "F.Cu") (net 10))
 (segment (start 116.205 81.915) (end 114.3 83.82) (width 0.4) (layer "F.Cu") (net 10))
 (segment (start 128.27 85.09) (end 129.54 83.82) (width 0.4) (layer "F.Cu") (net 9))
 (segment (start 116.84 83.82) (end 118.11 85.09) (width 0.4) (layer "F.Cu") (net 9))
 (segment (start 118.11 85.09) (end 128.27 85.09) (width 0.4) (layer "F.Cu") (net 9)))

